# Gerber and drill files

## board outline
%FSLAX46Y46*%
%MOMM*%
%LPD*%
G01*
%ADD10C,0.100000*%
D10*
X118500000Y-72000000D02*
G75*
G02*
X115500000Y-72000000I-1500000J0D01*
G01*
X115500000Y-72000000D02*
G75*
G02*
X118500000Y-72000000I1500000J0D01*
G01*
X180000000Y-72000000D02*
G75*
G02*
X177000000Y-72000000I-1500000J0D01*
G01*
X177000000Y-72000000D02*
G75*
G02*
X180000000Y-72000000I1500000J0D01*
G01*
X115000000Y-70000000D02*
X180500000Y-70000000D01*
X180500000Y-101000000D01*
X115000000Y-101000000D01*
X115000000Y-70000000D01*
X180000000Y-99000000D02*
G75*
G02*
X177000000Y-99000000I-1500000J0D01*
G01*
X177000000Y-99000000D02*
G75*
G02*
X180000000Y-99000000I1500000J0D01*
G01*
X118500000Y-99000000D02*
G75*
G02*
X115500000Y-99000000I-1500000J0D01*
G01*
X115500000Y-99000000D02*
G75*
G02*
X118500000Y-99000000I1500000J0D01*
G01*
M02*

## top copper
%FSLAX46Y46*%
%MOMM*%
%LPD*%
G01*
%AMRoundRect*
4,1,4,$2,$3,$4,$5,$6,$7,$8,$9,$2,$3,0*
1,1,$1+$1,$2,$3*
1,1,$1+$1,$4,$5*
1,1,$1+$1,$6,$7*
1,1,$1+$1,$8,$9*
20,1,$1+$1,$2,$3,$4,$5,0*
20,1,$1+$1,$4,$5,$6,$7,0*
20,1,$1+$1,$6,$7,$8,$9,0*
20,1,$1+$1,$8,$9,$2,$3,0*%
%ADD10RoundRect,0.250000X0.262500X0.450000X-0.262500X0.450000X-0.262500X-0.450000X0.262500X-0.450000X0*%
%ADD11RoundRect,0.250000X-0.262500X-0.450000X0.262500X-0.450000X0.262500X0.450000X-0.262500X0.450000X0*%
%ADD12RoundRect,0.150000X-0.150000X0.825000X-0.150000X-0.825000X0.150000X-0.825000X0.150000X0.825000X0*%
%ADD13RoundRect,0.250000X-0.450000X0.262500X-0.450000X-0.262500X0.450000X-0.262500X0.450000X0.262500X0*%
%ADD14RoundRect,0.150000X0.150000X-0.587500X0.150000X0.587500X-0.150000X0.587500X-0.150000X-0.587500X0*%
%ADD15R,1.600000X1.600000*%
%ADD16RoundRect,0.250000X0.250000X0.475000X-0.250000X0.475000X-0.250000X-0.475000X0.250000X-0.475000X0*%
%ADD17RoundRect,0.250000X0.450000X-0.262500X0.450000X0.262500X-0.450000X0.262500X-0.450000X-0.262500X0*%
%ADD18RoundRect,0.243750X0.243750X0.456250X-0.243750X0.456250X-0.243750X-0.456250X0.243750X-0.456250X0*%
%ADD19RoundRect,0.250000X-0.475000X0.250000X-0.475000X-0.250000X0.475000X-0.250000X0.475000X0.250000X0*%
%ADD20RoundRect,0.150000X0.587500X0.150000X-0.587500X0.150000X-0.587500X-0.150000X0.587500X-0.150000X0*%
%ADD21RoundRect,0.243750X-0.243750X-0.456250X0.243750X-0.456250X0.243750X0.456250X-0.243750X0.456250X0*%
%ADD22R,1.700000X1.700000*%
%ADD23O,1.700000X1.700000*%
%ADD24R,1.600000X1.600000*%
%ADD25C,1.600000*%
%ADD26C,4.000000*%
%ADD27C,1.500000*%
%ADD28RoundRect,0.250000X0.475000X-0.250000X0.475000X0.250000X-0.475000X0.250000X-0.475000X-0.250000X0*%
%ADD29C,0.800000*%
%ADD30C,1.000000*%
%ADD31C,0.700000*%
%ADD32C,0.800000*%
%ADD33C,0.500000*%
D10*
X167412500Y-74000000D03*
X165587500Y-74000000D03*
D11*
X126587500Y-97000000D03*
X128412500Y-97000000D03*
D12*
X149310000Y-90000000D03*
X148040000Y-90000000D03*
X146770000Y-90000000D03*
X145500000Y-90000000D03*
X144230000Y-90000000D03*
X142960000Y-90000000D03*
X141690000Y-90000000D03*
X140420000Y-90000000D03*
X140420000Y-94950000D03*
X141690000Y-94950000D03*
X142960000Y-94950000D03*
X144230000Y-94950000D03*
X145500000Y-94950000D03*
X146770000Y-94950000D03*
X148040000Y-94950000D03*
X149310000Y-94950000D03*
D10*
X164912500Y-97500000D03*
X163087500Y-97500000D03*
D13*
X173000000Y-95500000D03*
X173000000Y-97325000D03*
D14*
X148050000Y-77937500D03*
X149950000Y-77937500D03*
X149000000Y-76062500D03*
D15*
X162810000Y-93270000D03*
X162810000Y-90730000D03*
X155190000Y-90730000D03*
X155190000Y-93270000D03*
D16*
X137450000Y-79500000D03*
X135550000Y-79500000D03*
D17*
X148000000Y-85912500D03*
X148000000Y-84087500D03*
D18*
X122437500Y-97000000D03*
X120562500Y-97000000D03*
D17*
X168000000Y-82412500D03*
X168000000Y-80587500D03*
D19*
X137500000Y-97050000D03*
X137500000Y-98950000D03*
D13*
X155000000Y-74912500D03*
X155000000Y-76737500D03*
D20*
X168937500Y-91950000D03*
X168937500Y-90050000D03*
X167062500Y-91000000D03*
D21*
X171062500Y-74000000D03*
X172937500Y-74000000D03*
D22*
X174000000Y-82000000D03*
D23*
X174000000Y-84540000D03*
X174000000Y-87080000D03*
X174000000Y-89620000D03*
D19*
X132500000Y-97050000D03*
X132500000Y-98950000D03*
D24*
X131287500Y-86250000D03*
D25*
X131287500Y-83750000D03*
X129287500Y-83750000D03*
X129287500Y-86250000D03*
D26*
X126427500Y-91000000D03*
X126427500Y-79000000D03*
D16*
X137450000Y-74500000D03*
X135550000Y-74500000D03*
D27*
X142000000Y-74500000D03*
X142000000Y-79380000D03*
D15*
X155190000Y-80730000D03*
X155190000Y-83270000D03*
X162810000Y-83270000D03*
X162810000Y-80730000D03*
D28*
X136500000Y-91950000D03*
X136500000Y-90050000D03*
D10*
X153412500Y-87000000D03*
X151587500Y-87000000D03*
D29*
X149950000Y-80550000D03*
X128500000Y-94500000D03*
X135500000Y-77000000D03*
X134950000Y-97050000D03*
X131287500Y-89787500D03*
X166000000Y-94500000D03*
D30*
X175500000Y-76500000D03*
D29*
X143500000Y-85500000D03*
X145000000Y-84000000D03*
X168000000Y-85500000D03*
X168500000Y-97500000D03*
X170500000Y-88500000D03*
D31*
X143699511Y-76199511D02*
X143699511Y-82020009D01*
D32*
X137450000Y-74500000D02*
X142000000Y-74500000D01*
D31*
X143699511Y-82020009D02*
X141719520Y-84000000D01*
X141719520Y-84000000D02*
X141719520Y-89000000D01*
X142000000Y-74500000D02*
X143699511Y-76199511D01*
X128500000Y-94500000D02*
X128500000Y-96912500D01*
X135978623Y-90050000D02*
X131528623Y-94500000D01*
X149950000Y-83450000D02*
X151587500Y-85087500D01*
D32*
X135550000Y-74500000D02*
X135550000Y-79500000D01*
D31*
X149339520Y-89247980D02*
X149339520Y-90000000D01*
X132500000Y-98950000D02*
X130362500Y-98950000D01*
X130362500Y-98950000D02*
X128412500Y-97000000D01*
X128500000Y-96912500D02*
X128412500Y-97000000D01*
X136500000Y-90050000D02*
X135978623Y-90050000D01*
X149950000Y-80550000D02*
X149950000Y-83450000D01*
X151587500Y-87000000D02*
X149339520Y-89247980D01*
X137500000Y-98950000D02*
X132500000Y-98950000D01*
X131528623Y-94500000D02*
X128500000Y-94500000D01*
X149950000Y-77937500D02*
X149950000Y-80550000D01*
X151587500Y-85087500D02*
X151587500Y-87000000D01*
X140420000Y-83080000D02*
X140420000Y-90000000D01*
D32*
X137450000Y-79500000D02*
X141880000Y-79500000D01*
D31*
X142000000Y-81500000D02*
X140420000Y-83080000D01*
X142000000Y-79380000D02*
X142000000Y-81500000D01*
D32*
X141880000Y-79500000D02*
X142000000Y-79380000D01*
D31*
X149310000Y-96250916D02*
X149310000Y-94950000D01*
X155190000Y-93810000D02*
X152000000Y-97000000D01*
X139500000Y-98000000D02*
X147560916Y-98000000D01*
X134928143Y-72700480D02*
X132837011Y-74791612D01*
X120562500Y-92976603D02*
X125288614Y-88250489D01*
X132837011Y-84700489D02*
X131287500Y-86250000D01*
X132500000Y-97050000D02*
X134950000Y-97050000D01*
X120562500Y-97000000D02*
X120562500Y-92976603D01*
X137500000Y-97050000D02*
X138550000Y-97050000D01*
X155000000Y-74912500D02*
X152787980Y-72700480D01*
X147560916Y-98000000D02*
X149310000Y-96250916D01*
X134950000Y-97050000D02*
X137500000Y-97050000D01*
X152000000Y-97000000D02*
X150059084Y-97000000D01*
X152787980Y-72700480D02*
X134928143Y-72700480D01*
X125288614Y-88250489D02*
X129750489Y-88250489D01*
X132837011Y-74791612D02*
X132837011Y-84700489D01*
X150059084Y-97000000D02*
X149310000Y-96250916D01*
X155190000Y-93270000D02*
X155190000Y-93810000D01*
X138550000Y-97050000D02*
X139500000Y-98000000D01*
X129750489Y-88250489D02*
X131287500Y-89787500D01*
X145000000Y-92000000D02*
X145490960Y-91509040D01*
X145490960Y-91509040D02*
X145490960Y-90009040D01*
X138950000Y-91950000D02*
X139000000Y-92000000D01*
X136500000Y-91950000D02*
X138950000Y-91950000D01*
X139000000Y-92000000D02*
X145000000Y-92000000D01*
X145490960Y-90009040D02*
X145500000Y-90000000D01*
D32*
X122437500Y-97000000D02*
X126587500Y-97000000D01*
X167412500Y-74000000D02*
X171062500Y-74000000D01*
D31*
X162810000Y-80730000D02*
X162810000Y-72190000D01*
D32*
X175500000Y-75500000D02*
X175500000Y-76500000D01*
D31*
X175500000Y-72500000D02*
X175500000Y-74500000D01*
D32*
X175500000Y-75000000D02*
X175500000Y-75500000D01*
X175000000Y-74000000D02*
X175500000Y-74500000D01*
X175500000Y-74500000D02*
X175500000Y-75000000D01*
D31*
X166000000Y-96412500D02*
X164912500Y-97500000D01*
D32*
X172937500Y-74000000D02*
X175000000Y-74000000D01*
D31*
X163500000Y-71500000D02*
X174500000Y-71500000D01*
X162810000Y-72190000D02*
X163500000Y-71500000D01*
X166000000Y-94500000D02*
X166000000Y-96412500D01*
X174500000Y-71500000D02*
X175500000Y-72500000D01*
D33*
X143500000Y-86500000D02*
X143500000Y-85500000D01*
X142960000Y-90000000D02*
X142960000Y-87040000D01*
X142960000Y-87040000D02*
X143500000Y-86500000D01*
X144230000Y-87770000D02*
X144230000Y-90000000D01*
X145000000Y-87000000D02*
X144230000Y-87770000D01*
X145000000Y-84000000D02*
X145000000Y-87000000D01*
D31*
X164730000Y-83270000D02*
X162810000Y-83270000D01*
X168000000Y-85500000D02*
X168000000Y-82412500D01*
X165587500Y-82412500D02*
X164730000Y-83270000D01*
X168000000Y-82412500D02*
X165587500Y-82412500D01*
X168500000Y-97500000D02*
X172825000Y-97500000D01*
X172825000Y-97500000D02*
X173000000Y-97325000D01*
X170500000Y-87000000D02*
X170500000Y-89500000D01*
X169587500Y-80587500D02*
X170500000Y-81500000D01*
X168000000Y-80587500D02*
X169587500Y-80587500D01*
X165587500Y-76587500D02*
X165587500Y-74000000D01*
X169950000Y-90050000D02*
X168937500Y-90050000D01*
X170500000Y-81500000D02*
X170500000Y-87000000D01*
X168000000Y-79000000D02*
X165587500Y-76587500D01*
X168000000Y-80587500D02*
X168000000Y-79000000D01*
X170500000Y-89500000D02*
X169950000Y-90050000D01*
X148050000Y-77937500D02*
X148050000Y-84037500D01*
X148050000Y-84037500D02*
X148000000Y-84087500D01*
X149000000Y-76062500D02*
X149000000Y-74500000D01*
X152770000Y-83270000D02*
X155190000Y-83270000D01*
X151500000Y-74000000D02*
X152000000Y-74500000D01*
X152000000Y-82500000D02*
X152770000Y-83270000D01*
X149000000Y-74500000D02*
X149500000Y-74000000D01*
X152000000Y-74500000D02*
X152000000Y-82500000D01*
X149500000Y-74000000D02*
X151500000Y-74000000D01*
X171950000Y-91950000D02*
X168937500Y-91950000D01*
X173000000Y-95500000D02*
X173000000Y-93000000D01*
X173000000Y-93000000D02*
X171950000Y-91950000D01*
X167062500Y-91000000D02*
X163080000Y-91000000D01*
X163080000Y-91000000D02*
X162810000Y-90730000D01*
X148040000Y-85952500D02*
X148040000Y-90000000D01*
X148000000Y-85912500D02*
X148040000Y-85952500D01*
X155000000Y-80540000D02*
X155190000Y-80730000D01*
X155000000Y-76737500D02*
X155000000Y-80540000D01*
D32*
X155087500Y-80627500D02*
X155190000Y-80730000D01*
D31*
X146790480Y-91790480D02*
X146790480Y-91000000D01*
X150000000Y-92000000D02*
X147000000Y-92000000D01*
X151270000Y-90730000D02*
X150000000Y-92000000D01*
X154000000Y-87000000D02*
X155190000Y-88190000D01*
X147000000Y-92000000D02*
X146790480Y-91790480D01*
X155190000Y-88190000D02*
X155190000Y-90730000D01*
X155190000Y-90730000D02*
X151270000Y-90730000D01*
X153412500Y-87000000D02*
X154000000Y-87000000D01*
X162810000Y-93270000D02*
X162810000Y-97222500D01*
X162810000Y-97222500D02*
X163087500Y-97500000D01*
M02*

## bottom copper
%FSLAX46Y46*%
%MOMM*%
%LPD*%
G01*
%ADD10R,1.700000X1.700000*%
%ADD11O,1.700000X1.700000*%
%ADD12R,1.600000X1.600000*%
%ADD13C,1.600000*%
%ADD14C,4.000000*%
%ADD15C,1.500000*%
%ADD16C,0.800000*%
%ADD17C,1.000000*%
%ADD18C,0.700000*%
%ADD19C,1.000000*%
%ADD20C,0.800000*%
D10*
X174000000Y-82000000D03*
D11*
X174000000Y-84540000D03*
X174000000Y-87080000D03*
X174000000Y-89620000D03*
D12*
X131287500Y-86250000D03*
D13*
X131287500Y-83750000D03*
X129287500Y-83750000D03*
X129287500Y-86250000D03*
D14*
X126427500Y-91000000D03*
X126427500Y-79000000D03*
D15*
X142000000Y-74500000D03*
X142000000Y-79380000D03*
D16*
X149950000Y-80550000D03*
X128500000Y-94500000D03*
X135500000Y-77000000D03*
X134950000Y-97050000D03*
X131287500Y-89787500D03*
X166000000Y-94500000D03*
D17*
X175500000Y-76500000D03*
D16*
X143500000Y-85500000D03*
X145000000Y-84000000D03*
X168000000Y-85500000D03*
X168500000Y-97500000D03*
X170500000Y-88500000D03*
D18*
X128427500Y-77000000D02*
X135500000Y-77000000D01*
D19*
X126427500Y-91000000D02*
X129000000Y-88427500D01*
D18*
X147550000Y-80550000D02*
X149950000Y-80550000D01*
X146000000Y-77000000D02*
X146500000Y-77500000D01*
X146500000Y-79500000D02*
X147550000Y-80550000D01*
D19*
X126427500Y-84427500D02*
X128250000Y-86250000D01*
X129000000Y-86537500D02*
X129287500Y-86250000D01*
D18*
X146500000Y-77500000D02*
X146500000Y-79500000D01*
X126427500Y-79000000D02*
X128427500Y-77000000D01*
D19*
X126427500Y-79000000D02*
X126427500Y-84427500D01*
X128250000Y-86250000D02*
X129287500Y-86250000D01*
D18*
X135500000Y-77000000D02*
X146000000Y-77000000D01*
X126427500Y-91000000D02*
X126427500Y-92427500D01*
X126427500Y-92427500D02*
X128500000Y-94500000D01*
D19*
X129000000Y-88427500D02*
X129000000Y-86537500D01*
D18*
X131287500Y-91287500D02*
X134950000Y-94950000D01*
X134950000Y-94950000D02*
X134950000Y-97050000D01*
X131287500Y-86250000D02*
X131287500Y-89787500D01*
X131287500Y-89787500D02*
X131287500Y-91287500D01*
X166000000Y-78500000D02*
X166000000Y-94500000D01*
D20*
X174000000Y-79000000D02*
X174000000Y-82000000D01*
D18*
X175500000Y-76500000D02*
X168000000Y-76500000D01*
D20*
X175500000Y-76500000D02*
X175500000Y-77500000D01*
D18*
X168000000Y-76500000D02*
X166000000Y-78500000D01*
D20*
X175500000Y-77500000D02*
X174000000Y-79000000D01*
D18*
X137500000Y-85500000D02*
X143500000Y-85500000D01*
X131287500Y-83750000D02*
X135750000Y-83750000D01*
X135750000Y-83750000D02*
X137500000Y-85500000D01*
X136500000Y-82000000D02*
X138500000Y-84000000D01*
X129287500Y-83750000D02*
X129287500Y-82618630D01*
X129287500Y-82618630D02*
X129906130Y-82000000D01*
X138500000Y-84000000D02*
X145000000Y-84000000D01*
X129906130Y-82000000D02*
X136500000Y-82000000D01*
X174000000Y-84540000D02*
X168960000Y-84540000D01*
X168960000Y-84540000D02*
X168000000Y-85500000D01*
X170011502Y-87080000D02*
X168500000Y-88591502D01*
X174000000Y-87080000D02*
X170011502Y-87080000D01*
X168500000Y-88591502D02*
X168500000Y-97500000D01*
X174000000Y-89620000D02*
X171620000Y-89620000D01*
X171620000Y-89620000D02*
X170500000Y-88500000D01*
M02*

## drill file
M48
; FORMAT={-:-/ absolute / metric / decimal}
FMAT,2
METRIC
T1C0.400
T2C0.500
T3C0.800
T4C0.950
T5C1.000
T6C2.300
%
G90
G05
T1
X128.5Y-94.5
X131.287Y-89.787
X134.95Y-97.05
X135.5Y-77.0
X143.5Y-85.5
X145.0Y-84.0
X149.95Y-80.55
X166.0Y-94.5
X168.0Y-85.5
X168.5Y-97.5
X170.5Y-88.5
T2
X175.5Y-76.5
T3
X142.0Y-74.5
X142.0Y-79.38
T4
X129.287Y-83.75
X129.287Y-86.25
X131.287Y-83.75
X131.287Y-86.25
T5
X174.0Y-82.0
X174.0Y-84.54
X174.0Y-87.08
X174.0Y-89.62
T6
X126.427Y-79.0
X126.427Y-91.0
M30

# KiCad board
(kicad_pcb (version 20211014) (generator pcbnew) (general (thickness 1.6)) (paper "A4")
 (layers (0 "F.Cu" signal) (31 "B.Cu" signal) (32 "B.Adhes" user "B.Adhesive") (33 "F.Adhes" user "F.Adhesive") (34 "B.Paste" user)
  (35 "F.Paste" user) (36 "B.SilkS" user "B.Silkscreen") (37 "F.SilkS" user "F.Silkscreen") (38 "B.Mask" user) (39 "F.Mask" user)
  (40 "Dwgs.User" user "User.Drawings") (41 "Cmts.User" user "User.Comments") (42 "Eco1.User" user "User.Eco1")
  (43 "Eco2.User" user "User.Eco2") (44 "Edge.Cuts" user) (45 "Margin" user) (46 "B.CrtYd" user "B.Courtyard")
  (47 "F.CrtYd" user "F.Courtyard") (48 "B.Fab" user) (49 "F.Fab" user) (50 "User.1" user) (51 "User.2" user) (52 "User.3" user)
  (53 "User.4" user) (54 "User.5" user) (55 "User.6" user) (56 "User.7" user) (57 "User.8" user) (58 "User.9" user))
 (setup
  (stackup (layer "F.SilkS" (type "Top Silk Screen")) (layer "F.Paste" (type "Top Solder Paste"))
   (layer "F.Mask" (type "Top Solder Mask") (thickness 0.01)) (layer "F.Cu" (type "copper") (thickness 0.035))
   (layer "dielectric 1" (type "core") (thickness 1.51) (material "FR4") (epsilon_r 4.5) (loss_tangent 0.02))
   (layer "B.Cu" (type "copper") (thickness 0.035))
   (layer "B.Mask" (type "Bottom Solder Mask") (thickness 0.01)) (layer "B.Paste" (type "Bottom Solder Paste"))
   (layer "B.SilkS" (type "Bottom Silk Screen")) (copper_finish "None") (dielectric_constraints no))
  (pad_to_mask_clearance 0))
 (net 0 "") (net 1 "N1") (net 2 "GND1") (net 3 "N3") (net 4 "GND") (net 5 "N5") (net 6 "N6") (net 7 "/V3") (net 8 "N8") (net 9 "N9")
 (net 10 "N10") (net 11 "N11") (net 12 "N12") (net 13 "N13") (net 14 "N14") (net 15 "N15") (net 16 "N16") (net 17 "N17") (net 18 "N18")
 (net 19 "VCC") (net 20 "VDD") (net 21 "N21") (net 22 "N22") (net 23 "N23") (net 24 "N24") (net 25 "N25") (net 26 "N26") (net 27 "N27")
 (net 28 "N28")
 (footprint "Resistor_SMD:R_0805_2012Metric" (layer "F.Cu") (at 166.5 74 180)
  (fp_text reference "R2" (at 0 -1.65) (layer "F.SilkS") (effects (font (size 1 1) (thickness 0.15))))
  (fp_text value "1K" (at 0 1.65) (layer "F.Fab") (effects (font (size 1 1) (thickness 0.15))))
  (pad "1" smd roundrect (at -0.9125 0 180) (size 1.025 1.4) (layers "F.Cu" "F.Paste" "F.Mask") (roundrect_rratio 0.243902) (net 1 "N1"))
  (pad "2" smd roundrect (at 0.9125 0 180) (size 1.025 1.4) (layers "F.Cu" "F.Paste" "F.Mask") (roundrect_rratio 0.243902) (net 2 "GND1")))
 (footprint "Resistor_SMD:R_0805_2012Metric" (layer "F.Cu") (at 127.5 97)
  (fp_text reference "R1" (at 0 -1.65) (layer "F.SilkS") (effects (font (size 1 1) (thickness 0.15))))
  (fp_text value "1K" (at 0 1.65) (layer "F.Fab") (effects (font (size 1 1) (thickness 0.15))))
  (pad "1" smd roundrect (at -0.9125 0) (size 1.025 1.4) (layers "F.Cu" "F.Paste" "F.Mask") (roundrect_rratio 0.243902) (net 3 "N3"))
  (pad "2" smd roundrect (at 0.9125 0) (size 1.025 1.4) (layers "F.Cu" "F.Paste" "F.Mask") (roundrect_rratio 0.243902) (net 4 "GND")))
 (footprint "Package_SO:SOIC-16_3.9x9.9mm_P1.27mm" (layer "F.Cu") (at 144.865 92.475 -90)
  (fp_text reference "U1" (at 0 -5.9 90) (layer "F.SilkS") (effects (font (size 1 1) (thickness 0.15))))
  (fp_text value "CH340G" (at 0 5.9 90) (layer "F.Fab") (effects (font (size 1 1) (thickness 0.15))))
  (pad "1" smd roundrect (at -2.475 -4.445 270) (size 1.95 0.6) (layers "F.Cu" "F.Paste" "F.Mask") (roundrect_rratio 0.25) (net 4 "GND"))
  (pad "2" smd roundrect (at -2.475 -3.175 270) (size 1.95 0.6) (layers "F.Cu" "F.Paste" "F.Mask") (roundrect_rratio 0.25) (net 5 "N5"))
  (pad "3" smd roundrect (at -2.475 -1.905 270) (size 1.95 0.6) (layers "F.Cu" "F.Paste" "F.Mask") (roundrect_rratio 0.25) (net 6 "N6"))
  (pad "4" smd roundrect (at -2.475 -0.635 270) (size 1.95 0.6) (layers "F.Cu" "F.Paste" "F.Mask") (roundrect_rratio 0.25) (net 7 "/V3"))
  (pad "5" smd roundrect (at -2.475 0.635 270) (size 1.95 0.6) (layers "F.Cu" "F.Paste" "F.Mask") (roundrect_rratio 0.25) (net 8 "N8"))
  (pad "6" smd roundrect (at -2.475 1.905 270) (size 1.95 0.6) (layers "F.Cu" "F.Paste" "F.Mask") (roundrect_rratio 0.25) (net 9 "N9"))
  (pad "7" smd roundrect (at -2.475 3.175 270) (size 1.95 0.6) (layers "F.Cu" "F.Paste" "F.Mask") (roundrect_rratio 0.25) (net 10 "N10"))
  (pad "8" smd roundrect (at -2.475 4.445 270) (size 1.95 0.6) (layers "F.Cu" "F.Paste" "F.Mask") (roundrect_rratio 0.25) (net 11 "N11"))
  (pad "9" smd roundrect (at 2.475 4.445 270) (size 1.95 0.6) (layers "F.Cu" "F.Paste" "F.Mask") (roundrect_rratio 0.25) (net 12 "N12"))
  (pad "10" smd roundrect (at 2.475 3.175 270) (size 1.95 0.6) (layers "F.Cu" "F.Paste" "F.Mask") (roundrect_rratio 0.25) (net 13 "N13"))
  (pad "11" smd roundrect (at 2.475 1.905 270) (size 1.95 0.6) (layers "F.Cu" "F.Paste" "F.Mask") (roundrect_rratio 0.25) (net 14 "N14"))
  (pad "12" smd roundrect (at 2.475 0.635 270) (size 1.95 0.6) (layers "F.Cu" "F.Paste" "F.Mask") (roundrect_rratio 0.25) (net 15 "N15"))
  (pad "13" smd roundrect (at 2.475 -0.635 270) (size 1.95 0.6) (layers "F.Cu" "F.Paste" "F.Mask") (roundrect_rratio 0.25) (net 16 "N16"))
  (pad "14" smd roundrect (at 2.475 -1.905 270) (size 1.95 0.6) (layers "F.Cu" "F.Paste" "F.Mask") (roundrect_rratio 0.25) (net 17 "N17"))
  (pad "15" smd roundrect (at 2.475 -3.175 270) (size 1.95 0.6) (layers "F.Cu" "F.Paste" "F.Mask") (roundrect_rratio 0.25) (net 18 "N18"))
  (pad "16" smd roundrect (at 2.475 -4.445 270) (size 1.95 0.6) (layers "F.Cu" "F.Paste" "F.Mask") (roundrect_rratio 0.25) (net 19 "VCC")))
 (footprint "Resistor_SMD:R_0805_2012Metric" (layer "F.Cu") (at 164 97.5 180)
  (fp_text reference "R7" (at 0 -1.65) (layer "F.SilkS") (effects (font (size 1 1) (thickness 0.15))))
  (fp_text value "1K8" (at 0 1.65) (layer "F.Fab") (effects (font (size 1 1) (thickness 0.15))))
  (pad "1" smd roundrect (at -0.9125 0 180) (size 1.025 1.4) (layers "F.Cu" "F.Paste" "F.Mask") (roundrect_rratio 0.243902) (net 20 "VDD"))
  (pad "2" smd roundrect (at 0.9125 0 180) (size 1.025 1.4) (layers "F.Cu" "F.Paste" "F.Mask") (roundrect_rratio 0.243902) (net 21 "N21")))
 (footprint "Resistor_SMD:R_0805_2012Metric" (layer "F.Cu") (at 173 96.4125 -90)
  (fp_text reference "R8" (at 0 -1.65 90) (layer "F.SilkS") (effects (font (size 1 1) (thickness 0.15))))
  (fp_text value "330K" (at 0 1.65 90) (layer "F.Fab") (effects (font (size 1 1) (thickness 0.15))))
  (pad "1" smd roundrect (at -0.9125 0 270) (size 1.025 1.4) (layers "F.Cu" "F.Paste" "F.Mask") (roundrect_rratio 0.243902) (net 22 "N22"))
  (pad "2" smd roundrect (at 0.9125 0 270) (size 1.025 1.4) (layers "F.Cu" "F.Paste" "F.Mask") (roundrect_rratio 0.243902) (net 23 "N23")))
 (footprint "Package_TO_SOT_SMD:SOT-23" (layer "F.Cu") (at 149 77 90)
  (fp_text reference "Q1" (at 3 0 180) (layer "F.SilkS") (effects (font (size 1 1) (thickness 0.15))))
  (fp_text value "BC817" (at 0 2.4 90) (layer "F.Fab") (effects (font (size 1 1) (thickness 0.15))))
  (pad "1" smd roundrect (at -0.9375 -0.95 90) (size 1.475 0.6) (layers "F.Cu" "F.Paste" "F.Mask") (roundrect_rratio 0.25) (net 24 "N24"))
  (pad "2" smd roundrect (at -0.9375 0.95 90) (size 1.475 0.6) (layers "F.Cu" "F.Paste" "F.Mask") (roundrect_rratio 0.25) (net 4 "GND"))
  (pad "3" smd roundrect (at 0.9375 0 90) (size 1.475 0.6) (layers "F.Cu" "F.Paste" "F.Mask") (roundrect_rratio 0.25) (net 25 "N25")))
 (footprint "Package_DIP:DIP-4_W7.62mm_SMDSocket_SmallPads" (layer "F.Cu") (at 159 92 180)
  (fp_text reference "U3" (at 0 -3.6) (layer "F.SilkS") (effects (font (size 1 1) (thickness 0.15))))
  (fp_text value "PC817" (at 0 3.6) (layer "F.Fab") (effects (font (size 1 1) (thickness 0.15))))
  (pad "1" smd rect (at -3.81 -1.27 180) (size 1.6 1.6) (layers "F.Cu" "F.Paste" "F.Mask") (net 21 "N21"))
  (pad "2" smd rect (at -3.81 1.27 180) (size 1.6 1.6) (layers "F.Cu" "F.Paste" "F.Mask") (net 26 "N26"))
  (pad "3" smd rect (at 3.81 1.27 180) (size 1.6 1.6) (layers "F.Cu" "F.Paste" "F.Mask") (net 6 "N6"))
  (pad "4" smd rect (at 3.81 -1.27 180) (size 1.6 1.6) (layers "F.Cu" "F.Paste" "F.Mask") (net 19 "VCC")))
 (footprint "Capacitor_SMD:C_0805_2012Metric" (layer "F.Cu") (at 136.5 79.5 180)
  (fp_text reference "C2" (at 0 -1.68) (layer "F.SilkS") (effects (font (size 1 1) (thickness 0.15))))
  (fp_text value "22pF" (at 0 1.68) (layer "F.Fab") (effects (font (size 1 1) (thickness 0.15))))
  (pad "1" smd roundrect (at -0.95 0 180) (size 1 1.45) (layers "F.Cu" "F.Paste" "F.Mask") (roundrect_rratio 0.25) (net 11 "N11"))
  (pad "2" smd roundrect (at 0.95 0 180) (size 1 1.45) (layers "F.Cu" "F.Paste" "F.Mask") (roundrect_rratio 0.25) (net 4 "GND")))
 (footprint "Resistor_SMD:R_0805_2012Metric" (layer "F.Cu") (at 148 85 90)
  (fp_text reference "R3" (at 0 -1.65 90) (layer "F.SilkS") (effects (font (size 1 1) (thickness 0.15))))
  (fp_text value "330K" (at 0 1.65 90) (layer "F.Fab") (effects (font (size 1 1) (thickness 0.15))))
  (pad "1" smd roundrect (at -0.9125 0 90) (size 1.025 1.4) (layers "F.Cu" "F.Paste" "F.Mask") (roundrect_rratio 0.243902) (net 5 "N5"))
  (pad "2" smd roundrect (at 0.9125 0 90) (size 1.025 1.4) (layers "F.Cu" "F.Paste" "F.Mask") (roundrect_rratio 0.243902) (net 24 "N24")))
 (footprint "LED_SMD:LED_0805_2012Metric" (layer "F.Cu") (at 121.5 97 180)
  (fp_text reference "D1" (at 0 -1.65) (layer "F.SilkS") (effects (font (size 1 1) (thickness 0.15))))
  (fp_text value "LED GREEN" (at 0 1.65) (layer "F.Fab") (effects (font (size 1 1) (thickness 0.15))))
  (pad "1" smd roundrect (at -0.9375 0 180) (size 0.975 1.4) (layers "F.Cu" "F.Paste" "F.Mask") (roundrect_rratio 0.25) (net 3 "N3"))
  (pad "2" smd roundrect (at 0.9375 0 180) (size 0.975 1.4) (layers "F.Cu" "F.Paste" "F.Mask") (roundrect_rratio 0.25) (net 19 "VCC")))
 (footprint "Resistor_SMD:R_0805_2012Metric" (layer "F.Cu") (at 168 81.5 90)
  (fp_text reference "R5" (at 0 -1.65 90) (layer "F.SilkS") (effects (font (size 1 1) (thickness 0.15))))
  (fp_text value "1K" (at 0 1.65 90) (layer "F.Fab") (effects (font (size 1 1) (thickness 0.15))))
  (pad "1" smd roundrect (at -0.9125 0 90) (size 1.025 1.4) (layers "F.Cu" "F.Paste" "F.Mask") (roundrect_rratio 0.243902) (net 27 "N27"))
  (pad "2" smd roundrect (at 0.9125 0 90) (size 1.025 1.4) (layers "F.Cu" "F.Paste" "F.Mask") (roundrect_rratio 0.243902) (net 2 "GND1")))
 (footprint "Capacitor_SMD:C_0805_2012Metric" (layer "F.Cu") (at 137.5 98 -90)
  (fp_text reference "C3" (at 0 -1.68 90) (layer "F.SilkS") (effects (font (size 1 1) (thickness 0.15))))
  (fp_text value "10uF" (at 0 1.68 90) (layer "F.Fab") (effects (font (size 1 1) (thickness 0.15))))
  (pad "1" smd roundrect (at -0.95 0 270) (size 1 1.45) (layers "F.Cu" "F.Paste" "F.Mask") (roundrect_rratio 0.25) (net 19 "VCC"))
  (pad "2" smd roundrect (at 0.95 0 270) (size 1 1.45) (layers "F.Cu" "F.Paste" "F.Mask") (roundrect_rratio 0.25) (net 4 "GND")))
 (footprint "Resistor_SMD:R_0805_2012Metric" (layer "F.Cu") (at 155 75.825 -90)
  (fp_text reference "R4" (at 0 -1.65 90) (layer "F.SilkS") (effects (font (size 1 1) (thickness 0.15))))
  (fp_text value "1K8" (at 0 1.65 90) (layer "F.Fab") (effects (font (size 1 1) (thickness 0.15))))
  (pad "1" smd roundrect (at -0.9125 0 270) (size 1.025 1.4) (layers "F.Cu" "F.Paste" "F.Mask") (roundrect_rratio 0.243902) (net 19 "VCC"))
  (pad "2" smd roundrect (at 0.9125 0 270) (size 1.025 1.4) (layers "F.Cu" "F.Paste" "F.Mask") (roundrect_rratio 0.243902) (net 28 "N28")))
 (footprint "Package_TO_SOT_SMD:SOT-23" (layer "F.Cu") (at 168 91 180)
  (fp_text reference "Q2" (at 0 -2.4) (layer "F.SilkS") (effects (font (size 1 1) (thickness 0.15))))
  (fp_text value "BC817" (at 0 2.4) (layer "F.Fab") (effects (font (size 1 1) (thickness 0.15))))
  (pad "1" smd roundrect (at -0.9375 -0.95 180) (size 1.475 0.6) (layers "F.Cu" "F.Paste" "F.Mask") (roundrect_rratio 0.25) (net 22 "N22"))
  (pad "2" smd roundrect (at -0.9375 0.95 180) (size 1.475 0.6) (layers "F.Cu" "F.Paste" "F.Mask") (roundrect_rratio 0.25) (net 2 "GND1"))
  (pad "3" smd roundrect (at 0.9375 0 180) (size 1.475 0.6) (layers "F.Cu" "F.Paste" "F.Mask") (roundrect_rratio 0.25) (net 26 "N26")))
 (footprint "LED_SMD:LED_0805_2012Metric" (layer "F.Cu") (at 172 74)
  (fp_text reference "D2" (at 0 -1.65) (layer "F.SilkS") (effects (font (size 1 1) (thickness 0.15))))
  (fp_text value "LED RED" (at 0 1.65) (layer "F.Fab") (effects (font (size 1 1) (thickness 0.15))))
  (pad "1" smd roundrect (at -0.9375 0) (size 0.975 1.4) (layers "F.Cu" "F.Paste" "F.Mask") (roundrect_rratio 0.25) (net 1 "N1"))
  (pad "2" smd roundrect (at 0.9375 0) (size 0.975 1.4) (layers "F.Cu" "F.Paste" "F.Mask") (roundrect_rratio 0.25) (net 20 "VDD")))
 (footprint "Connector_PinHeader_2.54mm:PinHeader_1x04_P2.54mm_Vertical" (layer "F.Cu") (at 174 82)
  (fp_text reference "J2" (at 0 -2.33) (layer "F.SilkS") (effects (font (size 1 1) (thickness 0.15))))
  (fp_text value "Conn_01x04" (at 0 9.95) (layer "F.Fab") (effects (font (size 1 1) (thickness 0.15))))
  (pad "1" thru_hole rect (at 0 0) (size 1.7 1.7) (drill 1) (layers *.Cu *.Mask) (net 20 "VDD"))
  (pad "2" thru_hole oval (at 0 2.54) (size 1.7 1.7) (drill 1) (layers *.Cu *.Mask) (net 27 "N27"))
  (pad "3" thru_hole oval (at 0 5.08) (size 1.7 1.7) (drill 1) (layers *.Cu *.Mask) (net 23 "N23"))
  (pad "4" thru_hole oval (at 0 7.62) (size 1.7 1.7) (drill 1) (layers *.Cu *.Mask) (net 2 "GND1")))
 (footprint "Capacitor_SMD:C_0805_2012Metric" (layer "F.Cu") (at 132.5 98 -90)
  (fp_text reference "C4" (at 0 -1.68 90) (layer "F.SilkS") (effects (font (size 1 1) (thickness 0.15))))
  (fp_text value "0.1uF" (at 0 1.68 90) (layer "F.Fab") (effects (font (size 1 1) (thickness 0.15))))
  (pad "1" smd roundrect (at -0.95 0 270) (size 1 1.45) (layers "F.Cu" "F.Paste" "F.Mask") (roundrect_rratio 0.25) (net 19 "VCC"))
  (pad "2" smd roundrect (at 0.95 0 270) (size 1 1.45) (layers "F.Cu" "F.Paste" "F.Mask") (roundrect_rratio 0.25) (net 4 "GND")))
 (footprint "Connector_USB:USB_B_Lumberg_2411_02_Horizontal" (layer "F.Cu") (at 131.2875 86.25 180) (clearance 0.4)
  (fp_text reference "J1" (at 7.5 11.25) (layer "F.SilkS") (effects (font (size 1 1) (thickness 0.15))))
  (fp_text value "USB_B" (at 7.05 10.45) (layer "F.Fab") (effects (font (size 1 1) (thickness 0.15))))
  (pad "1" thru_hole rect (at 0 0 270) (size 1.6 1.6) (drill 0.95) (layers *.Cu *.Mask) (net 19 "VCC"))
  (pad "2" thru_hole circle (at 0 2.5 270) (size 1.6 1.6) (drill 0.95) (layers *.Cu *.Mask) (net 9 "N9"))
  (pad "3" thru_hole circle (at 2 2.5 270) (size 1.6 1.6) (drill 0.95) (layers *.Cu *.Mask) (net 8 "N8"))
  (pad "4" thru_hole circle (at 2 0 270) (size 1.6 1.6) (drill 0.95) (layers *.Cu *.Mask) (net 4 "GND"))
  (pad "5" thru_hole circle (at 4.86 -4.75 270) (size 4 4) (drill 2.3) (layers *.Cu *.Mask) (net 4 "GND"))
  (pad "5" thru_hole circle (at 4.86 7.25 270) (size 4 4) (drill 2.3) (layers *.Cu *.Mask) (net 4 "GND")))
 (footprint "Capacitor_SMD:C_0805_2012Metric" (layer "F.Cu") (at 136.5 74.5 180)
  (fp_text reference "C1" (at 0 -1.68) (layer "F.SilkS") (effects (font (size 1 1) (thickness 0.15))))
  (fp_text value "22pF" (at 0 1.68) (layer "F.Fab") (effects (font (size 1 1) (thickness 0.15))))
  (pad "1" smd roundrect (at -0.95 0 180) (size 1 1.45) (layers "F.Cu" "F.Paste" "F.Mask") (roundrect_rratio 0.25) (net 10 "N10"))
  (pad "2" smd roundrect (at 0.95 0 180) (size 1 1.45) (layers "F.Cu" "F.Paste" "F.Mask") (roundrect_rratio 0.25) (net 4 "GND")))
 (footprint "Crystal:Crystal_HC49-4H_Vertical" (layer "F.Cu") (at 142 74.5 -90)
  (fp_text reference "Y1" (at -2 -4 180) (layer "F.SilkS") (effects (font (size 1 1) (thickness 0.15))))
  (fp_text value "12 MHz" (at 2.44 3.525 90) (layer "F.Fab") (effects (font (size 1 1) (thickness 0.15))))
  (pad "1" thru_hole circle (at 0 0 270) (size 1.5 1.5) (drill 0.8) (layers *.Cu *.Mask) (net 10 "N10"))
  (pad "2" thru_hole circle (at 4.88 0 270) (size 1.5 1.5) (drill 0.8) (layers *.Cu *.Mask) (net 11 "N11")))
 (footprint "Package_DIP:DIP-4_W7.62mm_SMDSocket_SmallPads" (layer "F.Cu") (at 159 82)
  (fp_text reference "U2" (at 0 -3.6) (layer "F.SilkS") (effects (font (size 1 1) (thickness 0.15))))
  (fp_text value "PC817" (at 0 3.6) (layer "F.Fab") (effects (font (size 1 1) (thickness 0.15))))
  (pad "1" smd rect (at -3.81 -1.27) (size 1.6 1.6) (layers "F.Cu" "F.Paste" "F.Mask") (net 28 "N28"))
  (pad "2" smd rect (at -3.81 1.27) (size 1.6 1.6) (layers "F.Cu" "F.Paste" "F.Mask") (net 25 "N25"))
  (pad "3" smd rect (at 3.81 1.27) (size 1.6 1.6) (layers "F.Cu" "F.Paste" "F.Mask") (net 27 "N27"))
  (pad "4" smd rect (at 3.81 -1.27) (size 1.6 1.6) (layers "F.Cu" "F.Paste" "F.Mask") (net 20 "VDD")))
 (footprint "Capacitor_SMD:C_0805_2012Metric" (layer "F.Cu") (at 136.5 91 90)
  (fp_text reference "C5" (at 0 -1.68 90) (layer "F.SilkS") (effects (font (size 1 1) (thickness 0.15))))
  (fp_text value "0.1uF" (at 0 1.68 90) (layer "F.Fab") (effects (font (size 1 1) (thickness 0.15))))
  (pad "1" smd roundrect (at -0.95 0 90) (size 1 1.45) (layers "F.Cu" "F.Paste" "F.Mask") (roundrect_rratio 0.25) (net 7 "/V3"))
  (pad "2" smd roundrect (at 0.95 0 90) (size 1 1.45) (layers "F.Cu" "F.Paste" "F.Mask") (roundrect_rratio 0.25) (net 4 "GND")))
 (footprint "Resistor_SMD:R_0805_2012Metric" (layer "F.Cu") (at 152.5 87 180)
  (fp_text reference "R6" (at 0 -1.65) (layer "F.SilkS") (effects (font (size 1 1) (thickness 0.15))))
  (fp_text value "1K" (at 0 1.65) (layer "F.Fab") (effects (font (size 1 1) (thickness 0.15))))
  (pad "1" smd roundrect (at -0.9125 0 180) (size 1.025 1.4) (layers "F.Cu" "F.Paste" "F.Mask") (roundrect_rratio 0.243902) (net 6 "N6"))
  (pad "2" smd roundrect (at 0.9125 0 180) (size 1.025 1.4) (layers "F.Cu" "F.Paste" "F.Mask") (roundrect_rratio 0.243902) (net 4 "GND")))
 (gr_circle (center 117 72) (end 118.5 72) (layer "Edge.Cuts") (width 0.1) (fill none))
 (gr_circle (center 178.5 72) (end 180 72) (layer "Edge.Cuts") (width 0.1) (fill none))
 (gr_rect (start 115 70) (end 180.5 101) (layer "Edge.Cuts") (width 0.1) (fill none))
 (gr_circle (center 178.5 99) (end 180 99) (layer "Edge.Cuts") (width 0.1) (fill none))
 (gr_circle (center 117 99) (end 118.5 99) (layer "Edge.Cuts") (width 0.1) (fill none))
 (segment (start 143.699511 76.199511) (end 143.699511 82.020009) (width 0.7) (layer "F.Cu") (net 10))
 (segment (start 137.45 74.5) (end 142 74.5) (width 0.8) (layer "F.Cu") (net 10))
 (segment (start 143.699511 82.020009) (end 141.71952 84) (width 0.7) (layer "F.Cu") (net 10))
 (segment (start 141.71952 84) (end 141.71952 89) (width 0.7) (layer "F.Cu") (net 10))
 (segment (start 142 74.5) (end 143.699511 76.199511) (width 0.7) (layer "F.Cu") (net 10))
 (segment (start 128.5 94.5) (end 128.5 96.9125) (width 0.7) (layer "F.Cu") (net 4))
 (segment (start 135.978623 90.05) (end 131.528623 94.5) (width 0.7) (layer "F.Cu") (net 4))
 (segment (start 149.95 83.45) (end 151.5875 85.0875) (width 0.7) (layer "F.Cu") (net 4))
 (segment (start 135.55 74.5) (end 135.55 79.5) (width 0.8) (layer "F.Cu") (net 4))
 (segment (start 149.33952 89.24798) (end 149.33952 90) (width 0.7) (layer "F.Cu") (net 4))
 (segment (start 132.5 98.95) (end 130.3625 98.95) (width 0.7) (layer "F.Cu") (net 4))
 (segment (start 130.3625 98.95) (end 128.4125 97) (width 0.7) (layer "F.Cu") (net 4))
 (segment (start 128.5 96.9125) (end 128.4125 97) (width 0.7) (layer "F.Cu") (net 4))
 (segment (start 136.5 90.05) (end 135.978623 90.05) (width 0.7) (layer "F.Cu") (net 4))
 (segment (start 149.95 80.55) (end 149.95 83.45) (width 0.7) (layer "F.Cu") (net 4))
 (segment (start 151.5875 87) (end 149.33952 89.24798) (width 0.7) (layer "F.Cu") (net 4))
 (segment (start 137.5 98.95) (end 132.5 98.95) (width 0.7) (layer "F.Cu") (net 4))
 (segment (start 131.528623 94.5) (end 128.5 94.5) (width 0.7) (layer "F.Cu") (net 4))
 (segment (start 149.95 77.9375) (end 149.95 80.55) (width 0.7) (layer "F.Cu") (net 4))
 (segment (start 151.5875 85.0875) (end 151.5875 87) (width 0.7) (layer "F.Cu") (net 4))
 (via (at 149.95 80.55) (size 0.8) (drill 0.4) (layers "F.Cu" "B.Cu") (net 4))
 (via (at 128.5 94.5) (size 0.8) (drill 0.4) (layers "F.Cu" "B.Cu") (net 4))
 (via (at 135.5 77) (size 0.8) (drill 0.4) (layers "F.Cu" "B.Cu") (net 4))
 (segment (start 128.4275 77) (end 135.5 77) (width 0.7) (layer "B.Cu") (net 4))
 (segment (start 126.4275 91) (end 129 88.4275) (width 1) (layer "B.Cu") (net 4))
 (segment (start 147.55 80.55) (end 149.95 80.55) (width 0.7) (layer "B.Cu") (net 4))
 (segment (start 146 77) (end 146.5 77.5) (width 0.7) (layer "B.Cu") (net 4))
 (segment (start 146.5 79.5) (end 147.55 80.55) (width 0.7) (layer "B.Cu") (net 4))
 (segment (start 126.4275 84.4275) (end 128.25 86.25) (width 1) (layer "B.Cu") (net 4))
 (segment (start 129 86.5375) (end 129.2875 86.25) (width 1) (layer "B.Cu") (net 4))
 (segment (start 146.5 77.5) (end 146.5 79.5) (width 0.7) (layer "B.Cu") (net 4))
 (segment (start 126.4275 79) (end 128.4275 77) (width 0.7) (layer "B.Cu") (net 4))
 (segment (start 126.4275 79) (end 126.4275 84.4275) (width 1) (layer "B.Cu") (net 4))
 (segment (start 128.25 86.25) (end 129.2875 86.25) (width 1) (layer "B.Cu") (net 4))
 (segment (start 135.5 77) (end 146 77) (width 0.7) (layer "B.Cu") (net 4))
 (segment (start 126.4275 91) (end 126.4275 92.4275) (width 0.7) (layer "B.Cu") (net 4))
 (segment (start 126.4275 92.4275) (end 128.5 94.5) (width 0.7) (layer "B.Cu") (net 4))
 (segment (start 129 88.4275) (end 129 86.5375) (width 1) (layer "B.Cu") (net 4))
 (segment (start 140.42 83.08) (end 140.42 90) (width 0.7) (layer "F.Cu") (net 11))
 (segment (start 137.45 79.5) (end 141.88 79.5) (width 0.8) (layer "F.Cu") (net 11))
 (segment (start 142 81.5) (end 140.42 83.08) (width 0.7) (layer "F.Cu") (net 11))
 (segment (start 142 79.38) (end 142 81.5) (width 0.7) (layer "F.Cu") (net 11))
 (segment (start 141.88 79.5) (end 142 79.38) (width 0.8) (layer "F.Cu") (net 11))
 (segment (start 149.31 96.250916) (end 149.31 94.95) (width 0.7) (layer "F.Cu") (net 19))
 (segment (start 155.19 93.81) (end 152 97) (width 0.7) (layer "F.Cu") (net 19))
 (segment (start 139.5 98) (end 147.560916 98) (width 0.7) (layer "F.Cu") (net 19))
 (segment (start 134.928143 72.70048) (end 132.837011 74.791612) (width 0.7) (layer "F.Cu") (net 19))
 (segment (start 120.5625 92.976603) (end 125.288614 88.250489) (width 0.7) (layer "F.Cu") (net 19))
 (segment (start 132.837011 84.700489) (end 131.2875 86.25) (width 0.7) (layer "F.Cu") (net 19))
 (segment (start 132.5 97.05) (end 134.95 97.05) (width 0.7) (layer "F.Cu") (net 19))
 (segment (start 120.5625 97) (end 120.5625 92.976603) (width 0.7) (layer "F.Cu") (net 19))
 (segment (start 137.5 97.05) (end 138.55 97.05) (width 0.7) (layer "F.Cu") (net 19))
 (segment (start 155 74.9125) (end 152.78798 72.70048) (width 0.7) (layer "F.Cu") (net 19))
 (segment (start 147.560916 98) (end 149.31 96.250916) (width 0.7) (layer "F.Cu") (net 19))
 (segment (start 134.95 97.05) (end 137.5 97.05) (width 0.7) (layer "F.Cu") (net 19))
 (segment (start 152 97) (end 150.059084 97) (width 0.7) (layer "F.Cu") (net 19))
 (segment (start 152.78798 72.70048) (end 134.928143 72.70048) (width 0.7) (layer "F.Cu") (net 19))
 (segment (start 125.288614 88.250489) (end 129.750489 88.250489) (width 0.7) (layer "F.Cu") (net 19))
 (segment (start 132.837011 74.791612) (end 132.837011 84.700489) (width 0.7) (layer "F.Cu") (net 19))
 (segment (start 150.059084 97) (end 149.31 96.250916) (width 0.7) (layer "F.Cu") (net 19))
 (segment (start 155.19 93.27) (end 155.19 93.81) (width 0.7) (layer "F.Cu") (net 19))
 (segment (start 138.55 97.05) (end 139.5 98) (width 0.7) (layer "F.Cu") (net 19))
 (segment (start 129.750489 88.250489) (end 131.2875 89.7875) (width 0.7) (layer "F.Cu") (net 19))
 (via (at 134.95 97.05) (size 0.8) (drill 0.4) (layers "F.Cu" "B.Cu") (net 19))
 (via (at 131.2875 89.7875) (size 0.8) (drill 0.4) (layers "F.Cu" "B.Cu") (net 19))
 (segment (start 131.2875 91.2875) (end 134.95 94.95) (width 0.7) (layer "B.Cu") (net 19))
 (segment (start 134.95 94.95) (end 134.95 97.05) (width 0.7) (layer "B.Cu") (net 19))
 (segment (start 131.2875 86.25) (end 131.2875 89.7875) (width 0.7) (layer "B.Cu") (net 19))
 (segment (start 131.2875 89.7875) (end 131.2875 91.2875) (width 0.7) (layer "B.Cu") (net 19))
 (segment (start 145 92) (end 145.49096 91.50904) (width 0.7) (layer "F.Cu") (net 7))
 (segment (start 145.49096 91.50904) (end 145.49096 90.00904) (width 0.7) (layer "F.Cu") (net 7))
 (segment (start 138.95 91.95) (end 139 92) (width 0.7) (layer "F.Cu") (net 7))
 (segment (start 136.5 91.95) (end 138.95 91.95) (width 0.7) (layer "F.Cu") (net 7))
 (segment (start 139 92) (end 145 92) (width 0.7) (layer "F.Cu") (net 7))
 (segment (start 145.49096 90.00904) (end 145.5 90) (width 0.7) (layer "F.Cu") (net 7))
 (segment (start 122.4375 97) (end 126.5875 97) (width 0.8) (layer "F.Cu") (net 3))
 (segment (start 167.4125 74) (end 171.0625 74) (width 0.8) (layer "F.Cu") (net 1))
 (segment (start 162.81 80.73) (end 162.81 72.19) (width 0.7) (layer "F.Cu") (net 20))
 (segment (start 175.5 75.5) (end 175.5 76.5) (width 0.8) (layer "F.Cu") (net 20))
 (segment (start 175.5 72.5) (end 175.5 74.5) (width 0.7) (layer "F.Cu") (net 20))
 (segment (start 175.5 75) (end 175.5 75.5) (width 0.8) (layer "F.Cu") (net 20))
 (segment (start 175 74) (end 175.5 74.5) (width 0.8) (layer "F.Cu") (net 20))
 (segment (start 175.5 74.5) (end 175.5 75) (width 0.8) (layer "F.Cu") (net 20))
 (segment (start 166 96.4125) (end 164.9125 97.5) (width 0.7) (layer "F.Cu") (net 20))
 (segment (start 172.9375 74) (end 175 74) (width 0.8) (layer "F.Cu") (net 20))
 (segment (start 163.5 71.5) (end 174.5 71.5) (width 0.7) (layer "F.Cu") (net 20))
 (segment (start 162.81 72.19) (end 163.5 71.5) (width 0.7) (layer "F.Cu") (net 20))
 (segment (start 166 94.5) (end 166 96.4125) (width 0.7) (layer "F.Cu") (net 20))
 (segment (start 174.5 71.5) (end 175.5 72.5) (width 0.7) (layer "F.Cu") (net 20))
 (via (at 166 94.5) (size 0.8) (drill 0.4) (layers "F.Cu" "B.Cu") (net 20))
 (via (at 175.5 76.5) (size 1) (drill 0.5) (layers "F.Cu" "B.Cu") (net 20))
 (segment (start 166 78.5) (end 166 94.5) (width 0.7) (layer "B.Cu") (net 20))
 (segment (start 174 79) (end 174 82) (width 0.8) (layer "B.Cu") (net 20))
 (segment (start 175.5 76.5) (end 168 76.5) (width 0.7) (layer "B.Cu") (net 20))
 (segment (start 175.5 76.5) (end 175.5 77.5) (width 0.8) (layer "B.Cu") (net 20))
 (segment (start 168 76.5) (end 166 78.5) (width 0.7) (layer "B.Cu") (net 20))
 (segment (start 175.5 77.5) (end 174 79) (width 0.8) (layer "B.Cu") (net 20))
 (segment (start 143.5 86.5) (end 143.5 85.5) (width 0.5) (layer "F.Cu") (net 9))
 (segment (start 142.96 90) (end 142.96 87.04) (width 0.5) (layer "F.Cu") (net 9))
 (segment (start 142.96 87.04) (end 143.5 86.5) (width 0.5) (layer "F.Cu") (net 9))
 (via (at 143.5 85.5) (size 0.8) (drill 0.4) (layers "F.Cu" "B.Cu") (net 9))
 (segment (start 137.5 85.5) (end 143.5 85.5) (width 0.7) (layer "B.Cu") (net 9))
 (segment (start 131.2875 83.75) (end 135.75 83.75) (width 0.7) (layer "B.Cu") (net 9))
 (segment (start 135.75 83.75) (end 137.5 85.5) (width 0.7) (layer "B.Cu") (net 9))
 (segment (start 144.23 87.77) (end 144.23 90) (width 0.5) (layer "F.Cu") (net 8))
 (segment (start 145 87) (end 144.23 87.77) (width 0.5) (layer "F.Cu") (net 8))
 (segment (start 145 84) (end 145 87) (width 0.5) (layer "F.Cu") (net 8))
 (via (at 145 84) (size 0.8) (drill 0.4) (layers "F.Cu" "B.Cu") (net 8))
 (segment (start 136.5 82) (end 138.5 84) (width 0.7) (layer "B.Cu") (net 8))
 (segment (start 129.2875 83.75) (end 129.2875 82.61863) (width 0.7) (layer "B.Cu") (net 8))
 (segment (start 129.2875 82.61863) (end 129.90613 82) (width 0.7) (layer "B.Cu") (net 8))
 (segment (start 138.5 84) (end 145 84) (width 0.7) (layer "B.Cu") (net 8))
 (segment (start 129.90613 82) (end 136.5 82) (width 0.7) (layer "B.Cu") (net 8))
 (segment (start 164.73 83.27) (end 162.81 83.27) (width 0.7) (layer "F.Cu") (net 27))
 (segment (start 168 85.5) (end 168 82.4125) (width 0.7) (layer "F.Cu") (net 27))
 (segment (start 165.5875 82.4125) (end 164.73 83.27) (width 0.7) (layer "F.Cu") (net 27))
 (segment (start 168 82.4125) (end 165.5875 82.4125) (width 0.7) (layer "F.Cu") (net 27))
 (via (at 168 85.5) (size 0.8) (drill 0.4) (layers "F.Cu" "B.Cu") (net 27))
 (segment (start 174 84.54) (end 168.96 84.54) (width 0.7) (layer "B.Cu") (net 27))
 (segment (start 168.96 84.54) (end 168 85.5) (width 0.7) (layer "B.Cu") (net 27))
 (segment (start 168.5 97.5) (end 172.825 97.5) (width 0.7) (layer "F.Cu") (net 23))
 (segment (start 172.825 97.5) (end 173 97.325) (width 0.7) (layer "F.Cu") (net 23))
 (via (at 168.5 97.5) (size 0.8) (drill 0.4) (layers "F.Cu" "B.Cu") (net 23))
 (segment (start 170.011502 87.08) (end 168.5 88.591502) (width 0.7) (layer "B.Cu") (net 23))
 (segment (start 174 87.08) (end 170.011502 87.08) (width 0.7) (layer "B.Cu") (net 23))
 (segment (start 168.5 88.591502) (end 168.5 97.5) (width 0.7) (layer "B.Cu") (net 23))
 (segment (start 170.5 87) (end 170.5 89.5) (width 0.7) (layer "F.Cu") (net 2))
 (segment (start 169.5875 80.5875) (end 170.5 81.5) (width 0.7) (layer "F.Cu") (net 2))
 (segment (start 168 80.5875) (end 169.5875 80.5875) (width 0.7) (layer "F.Cu") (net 2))
 (segment (start 165.5875 76.5875) (end 165.5875 74) (width 0.7) (layer "F.Cu") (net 2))
 (segment (start 169.95 90.05) (end 168.9375 90.05) (width 0.7) (layer "F.Cu") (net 2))
 (segment (start 170.5 81.5) (end 170.5 87) (width 0.7) (layer "F.Cu") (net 2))
 (segment (start 168 79) (end 165.5875 76.5875) (width 0.7) (layer "F.Cu") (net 2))
 (segment (start 168 80.5875) (end 168 79) (width 0.7) (layer "F.Cu") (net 2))
 (segment (start 170.5 89.5) (end 169.95 90.05) (width 0.7) (layer "F.Cu") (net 2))
 (via (at 170.5 88.5) (size 0.8) (drill 0.4) (layers "F.Cu" "B.Cu") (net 2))
 (segment (start 174 89.62) (end 171.62 89.62) (width 0.7) (layer "B.Cu") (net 2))
 (segment (start 171.62 89.62) (end 170.5 88.5) (width 0.7) (layer "B.Cu") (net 2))
 (segment (start 148.05 77.9375) (end 148.05 84.0375) (width 0.7) (layer "F.Cu") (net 24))
 (segment (start 148.05 84.0375) (end 148 84.0875) (width 0.7) (layer "F.Cu") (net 24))
 (segment (start 149 76.0625) (end 149 74.5) (width 0.7) (layer "F.Cu") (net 25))
 (segment (start 152.77 83.27) (end 155.19 83.27) (width 0.7) (layer "F.Cu") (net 25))
 (segment (start 151.5 74) (end 152 74.5) (width 0.7) (layer "F.Cu") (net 25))
 (segment (start 152 82.5) (end 152.77 83.27) (width 0.7) (layer "F.Cu") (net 25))
 (segment (start 149 74.5) (end 149.5 74) (width 0.7) (layer "F.Cu") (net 25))
 (segment (start 152 74.5) (end 152 82.5) (width 0.7) (layer "F.Cu") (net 25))
 (segment (start 149.5 74) (end 151.5 74) (width 0.7) (layer "F.Cu") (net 25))
 (segment (start 171.95 91.95) (end 168.9375 91.95) (width 0.7) (layer "F.Cu") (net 22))
 (segment (start 173 95.5) (end 173 93) (width 0.7) (layer "F.Cu") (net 22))
 (segment (start 173 93) (end 171.95 91.95) (width 0.7) (layer "F.Cu") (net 22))
 (segment (start 167.0625 91) (end 163.08 91) (width 0.7) (layer "F.Cu") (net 26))
 (segment (start 163.08 91) (end 162.81 90.73) (width 0.7) (layer "F.Cu") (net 26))
 (segment (start 148.04 85.9525) (end 148.04 90) (width 0.7) (layer "F.Cu") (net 5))
 (segment (start 148 85.9125) (end 148.04 85.9525) (width 0.7) (layer "F.Cu") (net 5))
 (segment (start 155 80.54) (end 155.19 80.73) (width 0.7) (layer "F.Cu") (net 28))
 (segment (start 155 76.7375) (end 155 80.54) (width 0.7) (layer "F.Cu") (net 28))
 (segment (start 155.0875 80.6275) (end 155.19 80.73) (width 0.8) (layer "F.Cu") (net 28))
 (segment (start 146.79048 91.79048) (end 146.79048 91) (width 0.7) (layer "F.Cu") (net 6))
 (segment (start 150 92) (end 147 92) (width 0.7) (layer "F.Cu") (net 6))
 (segment (start 151.27 90.73) (end 150 92) (width 0.7) (layer "F.Cu") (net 6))
 (segment (start 154 87) (end 155.19 88.19) (width 0.7) (layer "F.Cu") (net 6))
 (segment (start 147 92) (end 146.79048 91.79048) (width 0.7) (layer "F.Cu") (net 6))
 (segment (start 155.19 88.19) (end 155.19 90.73) (width 0.7) (layer "F.Cu") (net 6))
 (segment (start 155.19 90.73) (end 151.27 90.73) (width 0.7) (layer "F.Cu") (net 6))
 (segment (start 153.4125 87) (end 154 87) (width 0.7) (layer "F.Cu") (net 6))
 (segment (start 162.81 93.27) (end 162.81 97.2225) (width 0.7) (layer "F.Cu") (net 21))
 (segment (start 162.81 97.2225) (end 163.0875 97.5) (width 0.7) (layer "F.Cu") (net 21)))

